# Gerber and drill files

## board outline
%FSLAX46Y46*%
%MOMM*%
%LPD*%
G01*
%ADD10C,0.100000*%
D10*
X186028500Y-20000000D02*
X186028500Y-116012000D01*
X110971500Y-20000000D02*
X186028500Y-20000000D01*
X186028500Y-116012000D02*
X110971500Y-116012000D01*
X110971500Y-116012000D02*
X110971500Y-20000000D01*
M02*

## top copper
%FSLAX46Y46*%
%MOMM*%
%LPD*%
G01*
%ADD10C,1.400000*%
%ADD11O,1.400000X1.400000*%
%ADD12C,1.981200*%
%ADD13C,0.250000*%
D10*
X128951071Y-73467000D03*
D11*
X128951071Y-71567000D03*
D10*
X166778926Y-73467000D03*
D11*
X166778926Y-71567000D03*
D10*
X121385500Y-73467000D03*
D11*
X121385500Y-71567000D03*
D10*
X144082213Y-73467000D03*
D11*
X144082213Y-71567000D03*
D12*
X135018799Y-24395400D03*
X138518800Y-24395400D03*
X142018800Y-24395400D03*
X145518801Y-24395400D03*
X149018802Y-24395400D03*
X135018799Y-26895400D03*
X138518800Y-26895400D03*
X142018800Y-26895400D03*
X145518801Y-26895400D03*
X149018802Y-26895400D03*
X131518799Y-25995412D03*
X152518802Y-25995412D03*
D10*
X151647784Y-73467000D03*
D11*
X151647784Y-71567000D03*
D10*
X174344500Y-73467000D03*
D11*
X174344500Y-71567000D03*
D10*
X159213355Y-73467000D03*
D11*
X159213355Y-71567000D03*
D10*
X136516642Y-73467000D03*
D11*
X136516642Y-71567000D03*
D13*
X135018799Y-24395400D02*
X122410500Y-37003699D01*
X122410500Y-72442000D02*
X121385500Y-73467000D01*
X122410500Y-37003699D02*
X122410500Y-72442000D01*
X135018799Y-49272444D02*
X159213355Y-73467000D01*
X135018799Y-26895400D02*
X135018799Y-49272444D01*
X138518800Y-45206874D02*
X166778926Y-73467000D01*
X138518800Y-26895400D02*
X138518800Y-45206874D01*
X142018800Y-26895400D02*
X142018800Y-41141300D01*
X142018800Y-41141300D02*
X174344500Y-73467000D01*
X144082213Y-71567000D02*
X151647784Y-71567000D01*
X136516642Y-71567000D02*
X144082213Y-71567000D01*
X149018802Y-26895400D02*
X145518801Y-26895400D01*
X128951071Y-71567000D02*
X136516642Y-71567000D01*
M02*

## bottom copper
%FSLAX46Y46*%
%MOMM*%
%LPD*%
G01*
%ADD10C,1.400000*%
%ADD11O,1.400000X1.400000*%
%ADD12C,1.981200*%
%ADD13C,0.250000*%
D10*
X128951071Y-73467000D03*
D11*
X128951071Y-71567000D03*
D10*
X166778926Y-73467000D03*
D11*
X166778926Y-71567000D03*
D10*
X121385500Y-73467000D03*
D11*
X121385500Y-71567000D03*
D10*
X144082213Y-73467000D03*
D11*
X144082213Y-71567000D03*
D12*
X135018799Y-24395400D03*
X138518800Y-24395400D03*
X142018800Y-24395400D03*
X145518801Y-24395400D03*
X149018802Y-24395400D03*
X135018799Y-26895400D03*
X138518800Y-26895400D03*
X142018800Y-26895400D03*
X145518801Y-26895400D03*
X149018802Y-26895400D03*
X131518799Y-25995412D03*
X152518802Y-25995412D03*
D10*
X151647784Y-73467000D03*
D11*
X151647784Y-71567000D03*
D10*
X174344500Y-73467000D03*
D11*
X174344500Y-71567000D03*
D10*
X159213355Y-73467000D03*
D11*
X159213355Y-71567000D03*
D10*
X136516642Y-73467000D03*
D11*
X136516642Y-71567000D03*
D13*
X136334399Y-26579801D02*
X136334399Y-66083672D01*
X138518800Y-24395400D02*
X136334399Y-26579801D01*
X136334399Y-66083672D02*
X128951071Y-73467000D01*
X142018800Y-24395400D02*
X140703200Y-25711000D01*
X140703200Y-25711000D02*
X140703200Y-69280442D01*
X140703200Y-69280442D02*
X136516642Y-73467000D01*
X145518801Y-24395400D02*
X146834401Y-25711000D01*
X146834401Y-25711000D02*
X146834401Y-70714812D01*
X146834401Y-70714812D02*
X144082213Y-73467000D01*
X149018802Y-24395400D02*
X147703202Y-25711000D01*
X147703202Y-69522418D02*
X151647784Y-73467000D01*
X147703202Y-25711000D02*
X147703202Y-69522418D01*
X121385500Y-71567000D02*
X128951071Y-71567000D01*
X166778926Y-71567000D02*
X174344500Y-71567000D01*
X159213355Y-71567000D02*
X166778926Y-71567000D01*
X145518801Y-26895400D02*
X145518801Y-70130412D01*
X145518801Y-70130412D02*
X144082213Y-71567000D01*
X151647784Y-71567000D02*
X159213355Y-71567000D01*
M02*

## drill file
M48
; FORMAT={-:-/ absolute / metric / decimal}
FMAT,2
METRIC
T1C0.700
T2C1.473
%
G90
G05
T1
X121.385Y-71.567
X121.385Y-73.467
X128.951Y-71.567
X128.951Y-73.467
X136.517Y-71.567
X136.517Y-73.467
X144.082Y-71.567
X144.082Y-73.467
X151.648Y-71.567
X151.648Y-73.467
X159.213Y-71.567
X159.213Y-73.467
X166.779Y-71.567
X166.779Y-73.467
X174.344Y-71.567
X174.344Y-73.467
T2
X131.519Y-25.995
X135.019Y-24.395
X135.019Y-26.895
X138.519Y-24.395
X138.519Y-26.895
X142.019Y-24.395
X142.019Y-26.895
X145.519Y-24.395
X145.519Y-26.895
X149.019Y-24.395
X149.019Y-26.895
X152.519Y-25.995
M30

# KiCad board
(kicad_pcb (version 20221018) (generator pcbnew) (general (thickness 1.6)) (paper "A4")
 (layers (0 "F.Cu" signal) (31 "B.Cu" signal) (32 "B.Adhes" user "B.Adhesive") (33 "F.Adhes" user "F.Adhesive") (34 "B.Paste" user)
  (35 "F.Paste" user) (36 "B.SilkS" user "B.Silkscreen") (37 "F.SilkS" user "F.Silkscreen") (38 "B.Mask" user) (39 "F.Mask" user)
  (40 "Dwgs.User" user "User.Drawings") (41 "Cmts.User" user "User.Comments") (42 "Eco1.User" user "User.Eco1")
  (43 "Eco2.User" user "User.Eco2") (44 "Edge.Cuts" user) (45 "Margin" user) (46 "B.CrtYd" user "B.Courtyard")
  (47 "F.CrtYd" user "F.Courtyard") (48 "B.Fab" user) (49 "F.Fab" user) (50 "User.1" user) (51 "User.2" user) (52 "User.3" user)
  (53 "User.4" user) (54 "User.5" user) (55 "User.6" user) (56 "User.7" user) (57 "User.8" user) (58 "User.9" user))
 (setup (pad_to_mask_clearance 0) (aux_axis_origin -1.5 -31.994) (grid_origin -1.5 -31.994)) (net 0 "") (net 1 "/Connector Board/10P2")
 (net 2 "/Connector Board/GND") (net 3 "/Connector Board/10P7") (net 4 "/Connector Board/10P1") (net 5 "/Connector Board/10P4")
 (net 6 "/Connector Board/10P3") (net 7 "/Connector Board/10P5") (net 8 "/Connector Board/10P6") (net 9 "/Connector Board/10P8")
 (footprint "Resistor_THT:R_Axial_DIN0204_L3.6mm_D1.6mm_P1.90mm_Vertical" (layer "F.Cu") (at 128.951071 73.467 90)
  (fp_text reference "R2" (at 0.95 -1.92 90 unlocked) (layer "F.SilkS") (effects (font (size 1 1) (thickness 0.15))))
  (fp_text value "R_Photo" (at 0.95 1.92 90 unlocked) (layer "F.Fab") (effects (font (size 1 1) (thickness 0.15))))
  (pad "1" thru_hole circle (at 0 0 90) (size 1.4 1.4) (drill 0.7) (layers "*.Cu" "*.Mask") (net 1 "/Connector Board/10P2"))
  (pad "2" thru_hole oval (at 1.9 0 90) (size 1.4 1.4) (drill 0.7) (layers "*.Cu" "*.Mask") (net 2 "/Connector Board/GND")))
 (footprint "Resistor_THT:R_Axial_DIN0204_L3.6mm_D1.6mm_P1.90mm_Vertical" (layer "F.Cu") (at 166.778926 73.467 90)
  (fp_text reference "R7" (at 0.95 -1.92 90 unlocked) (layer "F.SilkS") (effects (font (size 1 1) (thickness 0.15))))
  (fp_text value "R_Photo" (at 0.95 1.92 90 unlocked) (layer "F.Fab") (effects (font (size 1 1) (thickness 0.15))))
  (pad "1" thru_hole circle (at 0 0 90) (size 1.4 1.4) (drill 0.7) (layers "*.Cu" "*.Mask") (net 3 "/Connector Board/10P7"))
  (pad "2" thru_hole oval (at 1.9 0 90) (size 1.4 1.4) (drill 0.7) (layers "*.Cu" "*.Mask") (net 2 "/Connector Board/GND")))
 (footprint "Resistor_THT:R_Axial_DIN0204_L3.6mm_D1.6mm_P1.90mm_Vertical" (layer "F.Cu") (at 121.3855 73.467 90)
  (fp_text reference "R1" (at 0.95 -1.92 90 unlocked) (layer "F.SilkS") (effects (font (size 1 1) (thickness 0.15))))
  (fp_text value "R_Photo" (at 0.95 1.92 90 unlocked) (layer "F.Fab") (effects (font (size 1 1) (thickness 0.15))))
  (pad "1" thru_hole circle (at 0 0 90) (size 1.4 1.4) (drill 0.7) (layers "*.Cu" "*.Mask") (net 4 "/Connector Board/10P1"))
  (pad "2" thru_hole oval (at 1.9 0 90) (size 1.4 1.4) (drill 0.7) (layers "*.Cu" "*.Mask") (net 2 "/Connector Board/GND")))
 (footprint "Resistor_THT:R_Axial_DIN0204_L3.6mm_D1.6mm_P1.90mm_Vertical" (layer "F.Cu") (at 144.082213 73.467 90)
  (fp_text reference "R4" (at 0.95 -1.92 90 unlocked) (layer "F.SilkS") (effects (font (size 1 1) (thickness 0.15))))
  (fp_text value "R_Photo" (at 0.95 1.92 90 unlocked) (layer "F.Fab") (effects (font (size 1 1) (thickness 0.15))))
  (pad "1" thru_hole circle (at 0 0 90) (size 1.4 1.4) (drill 0.7) (layers "*.Cu" "*.Mask") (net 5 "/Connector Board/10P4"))
  (pad "2" thru_hole oval (at 1.9 0 90) (size 1.4 1.4) (drill 0.7) (layers "*.Cu" "*.Mask") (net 2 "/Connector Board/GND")))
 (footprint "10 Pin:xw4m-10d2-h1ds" (layer "F.Cu") (at 135.018799 24.3954)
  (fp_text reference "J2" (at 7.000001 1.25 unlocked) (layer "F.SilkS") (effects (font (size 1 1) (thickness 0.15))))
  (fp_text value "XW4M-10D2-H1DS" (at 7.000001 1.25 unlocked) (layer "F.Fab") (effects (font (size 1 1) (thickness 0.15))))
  (pad "1" thru_hole circle (at 0 0) (size 1.9812 1.9812) (drill 1.4732) (layers "*.Cu" "*.Mask") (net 4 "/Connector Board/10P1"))
  (pad "2" thru_hole circle (at 3.500001 0) (size 1.9812 1.9812) (drill 1.4732) (layers "*.Cu" "*.Mask") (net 1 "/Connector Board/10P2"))
  (pad "3" thru_hole circle (at 7.000001 0) (size 1.9812 1.9812) (drill 1.4732) (layers "*.Cu" "*.Mask") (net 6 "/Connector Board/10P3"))
  (pad "4" thru_hole circle (at 10.500002 0) (size 1.9812 1.9812) (drill 1.4732) (layers "*.Cu" "*.Mask") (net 5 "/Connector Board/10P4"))
  (pad "5" thru_hole circle (at 14.000003 0) (size 1.9812 1.9812) (drill 1.4732) (layers "*.Cu" "*.Mask") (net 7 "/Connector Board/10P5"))
  (pad "6" thru_hole circle (at 0 2.5) (size 1.9812 1.9812) (drill 1.4732) (layers "*.Cu" "*.Mask") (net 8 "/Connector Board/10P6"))
  (pad "7" thru_hole circle (at 3.500001 2.5) (size 1.9812 1.9812) (drill 1.4732) (layers "*.Cu" "*.Mask") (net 3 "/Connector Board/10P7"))
  (pad "8" thru_hole circle (at 7.000001 2.5) (size 1.9812 1.9812) (drill 1.4732) (layers "*.Cu" "*.Mask") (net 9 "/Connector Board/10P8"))
  (pad "9" thru_hole circle (at 10.500002 2.5) (size 1.9812 1.9812) (drill 1.4732) (layers "*.Cu" "*.Mask") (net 2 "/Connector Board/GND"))
  (pad "10" thru_hole circle (at 14.000003 2.5) (size 1.9812 1.9812) (drill 1.4732) (layers "*.Cu" "*.Mask") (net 2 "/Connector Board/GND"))
  (pad "11" thru_hole circle (at -3.5 1.600012) (size 1.9812 1.9812) (drill 1.4732) (layers "*.Cu" "*.Mask"))
  (pad "12" thru_hole circle (at 17.500003 1.600012) (size 1.9812 1.9812) (drill 1.4732) (layers "*.Cu" "*.Mask")))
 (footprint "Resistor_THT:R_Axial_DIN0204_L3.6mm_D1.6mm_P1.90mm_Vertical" (layer "F.Cu") (at 151.647784 73.467 90)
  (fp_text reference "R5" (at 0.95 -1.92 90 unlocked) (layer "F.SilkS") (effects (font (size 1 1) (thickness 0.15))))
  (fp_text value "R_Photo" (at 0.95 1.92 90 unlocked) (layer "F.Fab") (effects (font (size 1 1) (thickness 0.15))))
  (pad "1" thru_hole circle (at 0 0 90) (size 1.4 1.4) (drill 0.7) (layers "*.Cu" "*.Mask") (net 7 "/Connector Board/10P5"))
  (pad "2" thru_hole oval (at 1.9 0 90) (size 1.4 1.4) (drill 0.7) (layers "*.Cu" "*.Mask") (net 2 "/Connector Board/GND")))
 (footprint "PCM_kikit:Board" (layer "F.Cu") (at 111.2255 20)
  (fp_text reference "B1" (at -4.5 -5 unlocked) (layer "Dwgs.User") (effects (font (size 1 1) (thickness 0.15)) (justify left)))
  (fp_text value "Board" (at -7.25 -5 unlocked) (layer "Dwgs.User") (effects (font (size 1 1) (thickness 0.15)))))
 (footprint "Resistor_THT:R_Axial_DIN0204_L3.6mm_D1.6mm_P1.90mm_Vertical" (layer "F.Cu") (at 174.3445 73.467 90)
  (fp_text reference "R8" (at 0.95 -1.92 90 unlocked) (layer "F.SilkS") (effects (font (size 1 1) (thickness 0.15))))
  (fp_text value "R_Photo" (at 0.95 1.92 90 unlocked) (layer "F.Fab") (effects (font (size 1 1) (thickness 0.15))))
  (pad "1" thru_hole circle (at 0 0 90) (size 1.4 1.4) (drill 0.7) (layers "*.Cu" "*.Mask") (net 9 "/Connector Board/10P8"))
  (pad "2" thru_hole oval (at 1.9 0 90) (size 1.4 1.4) (drill 0.7) (layers "*.Cu" "*.Mask") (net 2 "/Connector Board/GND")))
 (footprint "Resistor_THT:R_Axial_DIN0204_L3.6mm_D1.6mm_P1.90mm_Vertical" (layer "F.Cu") (at 159.213355 73.467 90)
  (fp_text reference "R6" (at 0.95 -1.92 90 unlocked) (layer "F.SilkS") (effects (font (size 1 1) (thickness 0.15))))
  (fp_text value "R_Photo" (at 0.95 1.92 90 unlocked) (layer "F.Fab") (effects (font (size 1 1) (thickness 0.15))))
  (pad "1" thru_hole circle (at 0 0 90) (size 1.4 1.4) (drill 0.7) (layers "*.Cu" "*.Mask") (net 8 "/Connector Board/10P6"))
  (pad "2" thru_hole oval (at 1.9 0 90) (size 1.4 1.4) (drill 0.7) (layers "*.Cu" "*.Mask") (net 2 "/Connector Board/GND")))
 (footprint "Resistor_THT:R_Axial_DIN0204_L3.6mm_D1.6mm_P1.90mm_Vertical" (layer "F.Cu") (at 136.516642 73.467 90)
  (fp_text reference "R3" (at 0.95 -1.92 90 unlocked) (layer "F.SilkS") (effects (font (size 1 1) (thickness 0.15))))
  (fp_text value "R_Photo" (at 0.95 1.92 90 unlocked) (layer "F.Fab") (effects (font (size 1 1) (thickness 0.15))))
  (pad "1" thru_hole circle (at 0 0 90) (size 1.4 1.4) (drill 0.7) (layers "*.Cu" "*.Mask") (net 6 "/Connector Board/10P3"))
  (pad "2" thru_hole oval (at 1.9 0 90) (size 1.4 1.4) (drill 0.7) (layers "*.Cu" "*.Mask") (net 2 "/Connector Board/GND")))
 (gr_line (start 186.0285 20) (end 186.0285 116.012) (stroke (width 0.1) (type default)) (layer "Edge.Cuts"))
 (gr_line (start 110.9715 20) (end 186.0285 20) (stroke (width 0.1) (type default)) (layer "Edge.Cuts"))
 (gr_line (start 186.0285 116.012) (end 110.9715 116.012) (stroke (width 0.1) (type default)) (layer "Edge.Cuts"))
 (gr_line (start 110.9715 116.012) (end 110.9715 20) (stroke (width 0.1) (type default)) (layer "Edge.Cuts"))
 (segment (start 135.018799 24.3954) (end 122.4105 37.003699) (width 0.25) (layer "F.Cu") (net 4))
 (segment (start 122.4105 72.442) (end 121.3855 73.467) (width 0.25) (layer "F.Cu") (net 4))
 (segment (start 122.4105 37.003699) (end 122.4105 72.442) (width 0.25) (layer "F.Cu") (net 4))
 (segment (start 136.334399 26.579801) (end 136.334399 66.083672) (width 0.25) (layer "B.Cu") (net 1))
 (segment (start 138.5188 24.3954) (end 136.334399 26.579801) (width 0.25) (layer "B.Cu") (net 1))
 (segment (start 136.334399 66.083672) (end 128.951071 73.467) (width 0.25) (layer "B.Cu") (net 1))
 (segment (start 142.0188 24.3954) (end 140.7032 25.711) (width 0.25) (layer "B.Cu") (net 6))
 (segment (start 140.7032 25.711) (end 140.7032 69.280442) (width 0.25) (layer "B.Cu") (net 6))
 (segment (start 140.7032 69.280442) (end 136.516642 73.467) (width 0.25) (layer "B.Cu") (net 6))
 (segment (start 145.518801 24.3954) (end 146.834401 25.711) (width 0.25) (layer "B.Cu") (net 5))
 (segment (start 146.834401 25.711) (end 146.834401 70.714812) (width 0.25) (layer "B.Cu") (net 5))
 (segment (start 146.834401 70.714812) (end 144.082213 73.467) (width 0.25) (layer "B.Cu") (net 5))
 (segment (start 149.018802 24.3954) (end 147.703202 25.711) (width 0.25) (layer "B.Cu") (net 7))
 (segment (start 147.703202 69.522418) (end 151.647784 73.467) (width 0.25) (layer "B.Cu") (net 7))
 (segment (start 147.703202 25.711) (end 147.703202 69.522418) (width 0.25) (layer "B.Cu") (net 7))
 (segment (start 135.018799 49.272444) (end 159.213355 73.467) (width 0.25) (layer "F.Cu") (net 8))
 (segment (start 135.018799 26.8954) (end 135.018799 49.272444) (width 0.25) (layer "F.Cu") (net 8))
 (segment (start 138.5188 45.206874) (end 166.778926 73.467) (width 0.25) (layer "F.Cu") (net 3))
 (segment (start 138.5188 26.8954) (end 138.5188 45.206874) (width 0.25) (layer "F.Cu") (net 3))
 (segment (start 142.0188 26.8954) (end 142.0188 41.1413) (width 0.25) (layer "F.Cu") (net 9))
 (segment (start 142.0188 41.1413) (end 174.3445 73.467) (width 0.25) (layer "F.Cu") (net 9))
 (segment (start 144.082213 71.567) (end 151.647784 71.567) (width 0.25) (layer "F.Cu") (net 2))
 (segment (start 136.516642 71.567) (end 144.082213 71.567) (width 0.25) (layer "F.Cu") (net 2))
 (segment (start 149.018802 26.8954) (end 145.518801 26.8954) (width 0.25) (layer "F.Cu") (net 2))
 (segment (start 128.951071 71.567) (end 136.516642 71.567) (width 0.25) (layer "F.Cu") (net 2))
 (segment (start 121.3855 71.567) (end 128.951071 71.567) (width 0.25) (layer "B.Cu") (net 2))
 (segment (start 166.778926 71.567) (end 174.3445 71.567) (width 0.25) (layer "B.Cu") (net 2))
 (segment (start 159.213355 71.567) (end 166.778926 71.567) (width 0.25) (layer "B.Cu") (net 2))
 (segment (start 145.518801 26.8954) (end 145.518801 70.130412) (width 0.25) (layer "B.Cu") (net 2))
 (segment (start 145.518801 70.130412) (end 144.082213 71.567) (width 0.25) (layer "B.Cu") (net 2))
 (segment (start 151.647784 71.567) (end 159.213355 71.567) (width 0.25) (layer "B.Cu") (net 2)))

